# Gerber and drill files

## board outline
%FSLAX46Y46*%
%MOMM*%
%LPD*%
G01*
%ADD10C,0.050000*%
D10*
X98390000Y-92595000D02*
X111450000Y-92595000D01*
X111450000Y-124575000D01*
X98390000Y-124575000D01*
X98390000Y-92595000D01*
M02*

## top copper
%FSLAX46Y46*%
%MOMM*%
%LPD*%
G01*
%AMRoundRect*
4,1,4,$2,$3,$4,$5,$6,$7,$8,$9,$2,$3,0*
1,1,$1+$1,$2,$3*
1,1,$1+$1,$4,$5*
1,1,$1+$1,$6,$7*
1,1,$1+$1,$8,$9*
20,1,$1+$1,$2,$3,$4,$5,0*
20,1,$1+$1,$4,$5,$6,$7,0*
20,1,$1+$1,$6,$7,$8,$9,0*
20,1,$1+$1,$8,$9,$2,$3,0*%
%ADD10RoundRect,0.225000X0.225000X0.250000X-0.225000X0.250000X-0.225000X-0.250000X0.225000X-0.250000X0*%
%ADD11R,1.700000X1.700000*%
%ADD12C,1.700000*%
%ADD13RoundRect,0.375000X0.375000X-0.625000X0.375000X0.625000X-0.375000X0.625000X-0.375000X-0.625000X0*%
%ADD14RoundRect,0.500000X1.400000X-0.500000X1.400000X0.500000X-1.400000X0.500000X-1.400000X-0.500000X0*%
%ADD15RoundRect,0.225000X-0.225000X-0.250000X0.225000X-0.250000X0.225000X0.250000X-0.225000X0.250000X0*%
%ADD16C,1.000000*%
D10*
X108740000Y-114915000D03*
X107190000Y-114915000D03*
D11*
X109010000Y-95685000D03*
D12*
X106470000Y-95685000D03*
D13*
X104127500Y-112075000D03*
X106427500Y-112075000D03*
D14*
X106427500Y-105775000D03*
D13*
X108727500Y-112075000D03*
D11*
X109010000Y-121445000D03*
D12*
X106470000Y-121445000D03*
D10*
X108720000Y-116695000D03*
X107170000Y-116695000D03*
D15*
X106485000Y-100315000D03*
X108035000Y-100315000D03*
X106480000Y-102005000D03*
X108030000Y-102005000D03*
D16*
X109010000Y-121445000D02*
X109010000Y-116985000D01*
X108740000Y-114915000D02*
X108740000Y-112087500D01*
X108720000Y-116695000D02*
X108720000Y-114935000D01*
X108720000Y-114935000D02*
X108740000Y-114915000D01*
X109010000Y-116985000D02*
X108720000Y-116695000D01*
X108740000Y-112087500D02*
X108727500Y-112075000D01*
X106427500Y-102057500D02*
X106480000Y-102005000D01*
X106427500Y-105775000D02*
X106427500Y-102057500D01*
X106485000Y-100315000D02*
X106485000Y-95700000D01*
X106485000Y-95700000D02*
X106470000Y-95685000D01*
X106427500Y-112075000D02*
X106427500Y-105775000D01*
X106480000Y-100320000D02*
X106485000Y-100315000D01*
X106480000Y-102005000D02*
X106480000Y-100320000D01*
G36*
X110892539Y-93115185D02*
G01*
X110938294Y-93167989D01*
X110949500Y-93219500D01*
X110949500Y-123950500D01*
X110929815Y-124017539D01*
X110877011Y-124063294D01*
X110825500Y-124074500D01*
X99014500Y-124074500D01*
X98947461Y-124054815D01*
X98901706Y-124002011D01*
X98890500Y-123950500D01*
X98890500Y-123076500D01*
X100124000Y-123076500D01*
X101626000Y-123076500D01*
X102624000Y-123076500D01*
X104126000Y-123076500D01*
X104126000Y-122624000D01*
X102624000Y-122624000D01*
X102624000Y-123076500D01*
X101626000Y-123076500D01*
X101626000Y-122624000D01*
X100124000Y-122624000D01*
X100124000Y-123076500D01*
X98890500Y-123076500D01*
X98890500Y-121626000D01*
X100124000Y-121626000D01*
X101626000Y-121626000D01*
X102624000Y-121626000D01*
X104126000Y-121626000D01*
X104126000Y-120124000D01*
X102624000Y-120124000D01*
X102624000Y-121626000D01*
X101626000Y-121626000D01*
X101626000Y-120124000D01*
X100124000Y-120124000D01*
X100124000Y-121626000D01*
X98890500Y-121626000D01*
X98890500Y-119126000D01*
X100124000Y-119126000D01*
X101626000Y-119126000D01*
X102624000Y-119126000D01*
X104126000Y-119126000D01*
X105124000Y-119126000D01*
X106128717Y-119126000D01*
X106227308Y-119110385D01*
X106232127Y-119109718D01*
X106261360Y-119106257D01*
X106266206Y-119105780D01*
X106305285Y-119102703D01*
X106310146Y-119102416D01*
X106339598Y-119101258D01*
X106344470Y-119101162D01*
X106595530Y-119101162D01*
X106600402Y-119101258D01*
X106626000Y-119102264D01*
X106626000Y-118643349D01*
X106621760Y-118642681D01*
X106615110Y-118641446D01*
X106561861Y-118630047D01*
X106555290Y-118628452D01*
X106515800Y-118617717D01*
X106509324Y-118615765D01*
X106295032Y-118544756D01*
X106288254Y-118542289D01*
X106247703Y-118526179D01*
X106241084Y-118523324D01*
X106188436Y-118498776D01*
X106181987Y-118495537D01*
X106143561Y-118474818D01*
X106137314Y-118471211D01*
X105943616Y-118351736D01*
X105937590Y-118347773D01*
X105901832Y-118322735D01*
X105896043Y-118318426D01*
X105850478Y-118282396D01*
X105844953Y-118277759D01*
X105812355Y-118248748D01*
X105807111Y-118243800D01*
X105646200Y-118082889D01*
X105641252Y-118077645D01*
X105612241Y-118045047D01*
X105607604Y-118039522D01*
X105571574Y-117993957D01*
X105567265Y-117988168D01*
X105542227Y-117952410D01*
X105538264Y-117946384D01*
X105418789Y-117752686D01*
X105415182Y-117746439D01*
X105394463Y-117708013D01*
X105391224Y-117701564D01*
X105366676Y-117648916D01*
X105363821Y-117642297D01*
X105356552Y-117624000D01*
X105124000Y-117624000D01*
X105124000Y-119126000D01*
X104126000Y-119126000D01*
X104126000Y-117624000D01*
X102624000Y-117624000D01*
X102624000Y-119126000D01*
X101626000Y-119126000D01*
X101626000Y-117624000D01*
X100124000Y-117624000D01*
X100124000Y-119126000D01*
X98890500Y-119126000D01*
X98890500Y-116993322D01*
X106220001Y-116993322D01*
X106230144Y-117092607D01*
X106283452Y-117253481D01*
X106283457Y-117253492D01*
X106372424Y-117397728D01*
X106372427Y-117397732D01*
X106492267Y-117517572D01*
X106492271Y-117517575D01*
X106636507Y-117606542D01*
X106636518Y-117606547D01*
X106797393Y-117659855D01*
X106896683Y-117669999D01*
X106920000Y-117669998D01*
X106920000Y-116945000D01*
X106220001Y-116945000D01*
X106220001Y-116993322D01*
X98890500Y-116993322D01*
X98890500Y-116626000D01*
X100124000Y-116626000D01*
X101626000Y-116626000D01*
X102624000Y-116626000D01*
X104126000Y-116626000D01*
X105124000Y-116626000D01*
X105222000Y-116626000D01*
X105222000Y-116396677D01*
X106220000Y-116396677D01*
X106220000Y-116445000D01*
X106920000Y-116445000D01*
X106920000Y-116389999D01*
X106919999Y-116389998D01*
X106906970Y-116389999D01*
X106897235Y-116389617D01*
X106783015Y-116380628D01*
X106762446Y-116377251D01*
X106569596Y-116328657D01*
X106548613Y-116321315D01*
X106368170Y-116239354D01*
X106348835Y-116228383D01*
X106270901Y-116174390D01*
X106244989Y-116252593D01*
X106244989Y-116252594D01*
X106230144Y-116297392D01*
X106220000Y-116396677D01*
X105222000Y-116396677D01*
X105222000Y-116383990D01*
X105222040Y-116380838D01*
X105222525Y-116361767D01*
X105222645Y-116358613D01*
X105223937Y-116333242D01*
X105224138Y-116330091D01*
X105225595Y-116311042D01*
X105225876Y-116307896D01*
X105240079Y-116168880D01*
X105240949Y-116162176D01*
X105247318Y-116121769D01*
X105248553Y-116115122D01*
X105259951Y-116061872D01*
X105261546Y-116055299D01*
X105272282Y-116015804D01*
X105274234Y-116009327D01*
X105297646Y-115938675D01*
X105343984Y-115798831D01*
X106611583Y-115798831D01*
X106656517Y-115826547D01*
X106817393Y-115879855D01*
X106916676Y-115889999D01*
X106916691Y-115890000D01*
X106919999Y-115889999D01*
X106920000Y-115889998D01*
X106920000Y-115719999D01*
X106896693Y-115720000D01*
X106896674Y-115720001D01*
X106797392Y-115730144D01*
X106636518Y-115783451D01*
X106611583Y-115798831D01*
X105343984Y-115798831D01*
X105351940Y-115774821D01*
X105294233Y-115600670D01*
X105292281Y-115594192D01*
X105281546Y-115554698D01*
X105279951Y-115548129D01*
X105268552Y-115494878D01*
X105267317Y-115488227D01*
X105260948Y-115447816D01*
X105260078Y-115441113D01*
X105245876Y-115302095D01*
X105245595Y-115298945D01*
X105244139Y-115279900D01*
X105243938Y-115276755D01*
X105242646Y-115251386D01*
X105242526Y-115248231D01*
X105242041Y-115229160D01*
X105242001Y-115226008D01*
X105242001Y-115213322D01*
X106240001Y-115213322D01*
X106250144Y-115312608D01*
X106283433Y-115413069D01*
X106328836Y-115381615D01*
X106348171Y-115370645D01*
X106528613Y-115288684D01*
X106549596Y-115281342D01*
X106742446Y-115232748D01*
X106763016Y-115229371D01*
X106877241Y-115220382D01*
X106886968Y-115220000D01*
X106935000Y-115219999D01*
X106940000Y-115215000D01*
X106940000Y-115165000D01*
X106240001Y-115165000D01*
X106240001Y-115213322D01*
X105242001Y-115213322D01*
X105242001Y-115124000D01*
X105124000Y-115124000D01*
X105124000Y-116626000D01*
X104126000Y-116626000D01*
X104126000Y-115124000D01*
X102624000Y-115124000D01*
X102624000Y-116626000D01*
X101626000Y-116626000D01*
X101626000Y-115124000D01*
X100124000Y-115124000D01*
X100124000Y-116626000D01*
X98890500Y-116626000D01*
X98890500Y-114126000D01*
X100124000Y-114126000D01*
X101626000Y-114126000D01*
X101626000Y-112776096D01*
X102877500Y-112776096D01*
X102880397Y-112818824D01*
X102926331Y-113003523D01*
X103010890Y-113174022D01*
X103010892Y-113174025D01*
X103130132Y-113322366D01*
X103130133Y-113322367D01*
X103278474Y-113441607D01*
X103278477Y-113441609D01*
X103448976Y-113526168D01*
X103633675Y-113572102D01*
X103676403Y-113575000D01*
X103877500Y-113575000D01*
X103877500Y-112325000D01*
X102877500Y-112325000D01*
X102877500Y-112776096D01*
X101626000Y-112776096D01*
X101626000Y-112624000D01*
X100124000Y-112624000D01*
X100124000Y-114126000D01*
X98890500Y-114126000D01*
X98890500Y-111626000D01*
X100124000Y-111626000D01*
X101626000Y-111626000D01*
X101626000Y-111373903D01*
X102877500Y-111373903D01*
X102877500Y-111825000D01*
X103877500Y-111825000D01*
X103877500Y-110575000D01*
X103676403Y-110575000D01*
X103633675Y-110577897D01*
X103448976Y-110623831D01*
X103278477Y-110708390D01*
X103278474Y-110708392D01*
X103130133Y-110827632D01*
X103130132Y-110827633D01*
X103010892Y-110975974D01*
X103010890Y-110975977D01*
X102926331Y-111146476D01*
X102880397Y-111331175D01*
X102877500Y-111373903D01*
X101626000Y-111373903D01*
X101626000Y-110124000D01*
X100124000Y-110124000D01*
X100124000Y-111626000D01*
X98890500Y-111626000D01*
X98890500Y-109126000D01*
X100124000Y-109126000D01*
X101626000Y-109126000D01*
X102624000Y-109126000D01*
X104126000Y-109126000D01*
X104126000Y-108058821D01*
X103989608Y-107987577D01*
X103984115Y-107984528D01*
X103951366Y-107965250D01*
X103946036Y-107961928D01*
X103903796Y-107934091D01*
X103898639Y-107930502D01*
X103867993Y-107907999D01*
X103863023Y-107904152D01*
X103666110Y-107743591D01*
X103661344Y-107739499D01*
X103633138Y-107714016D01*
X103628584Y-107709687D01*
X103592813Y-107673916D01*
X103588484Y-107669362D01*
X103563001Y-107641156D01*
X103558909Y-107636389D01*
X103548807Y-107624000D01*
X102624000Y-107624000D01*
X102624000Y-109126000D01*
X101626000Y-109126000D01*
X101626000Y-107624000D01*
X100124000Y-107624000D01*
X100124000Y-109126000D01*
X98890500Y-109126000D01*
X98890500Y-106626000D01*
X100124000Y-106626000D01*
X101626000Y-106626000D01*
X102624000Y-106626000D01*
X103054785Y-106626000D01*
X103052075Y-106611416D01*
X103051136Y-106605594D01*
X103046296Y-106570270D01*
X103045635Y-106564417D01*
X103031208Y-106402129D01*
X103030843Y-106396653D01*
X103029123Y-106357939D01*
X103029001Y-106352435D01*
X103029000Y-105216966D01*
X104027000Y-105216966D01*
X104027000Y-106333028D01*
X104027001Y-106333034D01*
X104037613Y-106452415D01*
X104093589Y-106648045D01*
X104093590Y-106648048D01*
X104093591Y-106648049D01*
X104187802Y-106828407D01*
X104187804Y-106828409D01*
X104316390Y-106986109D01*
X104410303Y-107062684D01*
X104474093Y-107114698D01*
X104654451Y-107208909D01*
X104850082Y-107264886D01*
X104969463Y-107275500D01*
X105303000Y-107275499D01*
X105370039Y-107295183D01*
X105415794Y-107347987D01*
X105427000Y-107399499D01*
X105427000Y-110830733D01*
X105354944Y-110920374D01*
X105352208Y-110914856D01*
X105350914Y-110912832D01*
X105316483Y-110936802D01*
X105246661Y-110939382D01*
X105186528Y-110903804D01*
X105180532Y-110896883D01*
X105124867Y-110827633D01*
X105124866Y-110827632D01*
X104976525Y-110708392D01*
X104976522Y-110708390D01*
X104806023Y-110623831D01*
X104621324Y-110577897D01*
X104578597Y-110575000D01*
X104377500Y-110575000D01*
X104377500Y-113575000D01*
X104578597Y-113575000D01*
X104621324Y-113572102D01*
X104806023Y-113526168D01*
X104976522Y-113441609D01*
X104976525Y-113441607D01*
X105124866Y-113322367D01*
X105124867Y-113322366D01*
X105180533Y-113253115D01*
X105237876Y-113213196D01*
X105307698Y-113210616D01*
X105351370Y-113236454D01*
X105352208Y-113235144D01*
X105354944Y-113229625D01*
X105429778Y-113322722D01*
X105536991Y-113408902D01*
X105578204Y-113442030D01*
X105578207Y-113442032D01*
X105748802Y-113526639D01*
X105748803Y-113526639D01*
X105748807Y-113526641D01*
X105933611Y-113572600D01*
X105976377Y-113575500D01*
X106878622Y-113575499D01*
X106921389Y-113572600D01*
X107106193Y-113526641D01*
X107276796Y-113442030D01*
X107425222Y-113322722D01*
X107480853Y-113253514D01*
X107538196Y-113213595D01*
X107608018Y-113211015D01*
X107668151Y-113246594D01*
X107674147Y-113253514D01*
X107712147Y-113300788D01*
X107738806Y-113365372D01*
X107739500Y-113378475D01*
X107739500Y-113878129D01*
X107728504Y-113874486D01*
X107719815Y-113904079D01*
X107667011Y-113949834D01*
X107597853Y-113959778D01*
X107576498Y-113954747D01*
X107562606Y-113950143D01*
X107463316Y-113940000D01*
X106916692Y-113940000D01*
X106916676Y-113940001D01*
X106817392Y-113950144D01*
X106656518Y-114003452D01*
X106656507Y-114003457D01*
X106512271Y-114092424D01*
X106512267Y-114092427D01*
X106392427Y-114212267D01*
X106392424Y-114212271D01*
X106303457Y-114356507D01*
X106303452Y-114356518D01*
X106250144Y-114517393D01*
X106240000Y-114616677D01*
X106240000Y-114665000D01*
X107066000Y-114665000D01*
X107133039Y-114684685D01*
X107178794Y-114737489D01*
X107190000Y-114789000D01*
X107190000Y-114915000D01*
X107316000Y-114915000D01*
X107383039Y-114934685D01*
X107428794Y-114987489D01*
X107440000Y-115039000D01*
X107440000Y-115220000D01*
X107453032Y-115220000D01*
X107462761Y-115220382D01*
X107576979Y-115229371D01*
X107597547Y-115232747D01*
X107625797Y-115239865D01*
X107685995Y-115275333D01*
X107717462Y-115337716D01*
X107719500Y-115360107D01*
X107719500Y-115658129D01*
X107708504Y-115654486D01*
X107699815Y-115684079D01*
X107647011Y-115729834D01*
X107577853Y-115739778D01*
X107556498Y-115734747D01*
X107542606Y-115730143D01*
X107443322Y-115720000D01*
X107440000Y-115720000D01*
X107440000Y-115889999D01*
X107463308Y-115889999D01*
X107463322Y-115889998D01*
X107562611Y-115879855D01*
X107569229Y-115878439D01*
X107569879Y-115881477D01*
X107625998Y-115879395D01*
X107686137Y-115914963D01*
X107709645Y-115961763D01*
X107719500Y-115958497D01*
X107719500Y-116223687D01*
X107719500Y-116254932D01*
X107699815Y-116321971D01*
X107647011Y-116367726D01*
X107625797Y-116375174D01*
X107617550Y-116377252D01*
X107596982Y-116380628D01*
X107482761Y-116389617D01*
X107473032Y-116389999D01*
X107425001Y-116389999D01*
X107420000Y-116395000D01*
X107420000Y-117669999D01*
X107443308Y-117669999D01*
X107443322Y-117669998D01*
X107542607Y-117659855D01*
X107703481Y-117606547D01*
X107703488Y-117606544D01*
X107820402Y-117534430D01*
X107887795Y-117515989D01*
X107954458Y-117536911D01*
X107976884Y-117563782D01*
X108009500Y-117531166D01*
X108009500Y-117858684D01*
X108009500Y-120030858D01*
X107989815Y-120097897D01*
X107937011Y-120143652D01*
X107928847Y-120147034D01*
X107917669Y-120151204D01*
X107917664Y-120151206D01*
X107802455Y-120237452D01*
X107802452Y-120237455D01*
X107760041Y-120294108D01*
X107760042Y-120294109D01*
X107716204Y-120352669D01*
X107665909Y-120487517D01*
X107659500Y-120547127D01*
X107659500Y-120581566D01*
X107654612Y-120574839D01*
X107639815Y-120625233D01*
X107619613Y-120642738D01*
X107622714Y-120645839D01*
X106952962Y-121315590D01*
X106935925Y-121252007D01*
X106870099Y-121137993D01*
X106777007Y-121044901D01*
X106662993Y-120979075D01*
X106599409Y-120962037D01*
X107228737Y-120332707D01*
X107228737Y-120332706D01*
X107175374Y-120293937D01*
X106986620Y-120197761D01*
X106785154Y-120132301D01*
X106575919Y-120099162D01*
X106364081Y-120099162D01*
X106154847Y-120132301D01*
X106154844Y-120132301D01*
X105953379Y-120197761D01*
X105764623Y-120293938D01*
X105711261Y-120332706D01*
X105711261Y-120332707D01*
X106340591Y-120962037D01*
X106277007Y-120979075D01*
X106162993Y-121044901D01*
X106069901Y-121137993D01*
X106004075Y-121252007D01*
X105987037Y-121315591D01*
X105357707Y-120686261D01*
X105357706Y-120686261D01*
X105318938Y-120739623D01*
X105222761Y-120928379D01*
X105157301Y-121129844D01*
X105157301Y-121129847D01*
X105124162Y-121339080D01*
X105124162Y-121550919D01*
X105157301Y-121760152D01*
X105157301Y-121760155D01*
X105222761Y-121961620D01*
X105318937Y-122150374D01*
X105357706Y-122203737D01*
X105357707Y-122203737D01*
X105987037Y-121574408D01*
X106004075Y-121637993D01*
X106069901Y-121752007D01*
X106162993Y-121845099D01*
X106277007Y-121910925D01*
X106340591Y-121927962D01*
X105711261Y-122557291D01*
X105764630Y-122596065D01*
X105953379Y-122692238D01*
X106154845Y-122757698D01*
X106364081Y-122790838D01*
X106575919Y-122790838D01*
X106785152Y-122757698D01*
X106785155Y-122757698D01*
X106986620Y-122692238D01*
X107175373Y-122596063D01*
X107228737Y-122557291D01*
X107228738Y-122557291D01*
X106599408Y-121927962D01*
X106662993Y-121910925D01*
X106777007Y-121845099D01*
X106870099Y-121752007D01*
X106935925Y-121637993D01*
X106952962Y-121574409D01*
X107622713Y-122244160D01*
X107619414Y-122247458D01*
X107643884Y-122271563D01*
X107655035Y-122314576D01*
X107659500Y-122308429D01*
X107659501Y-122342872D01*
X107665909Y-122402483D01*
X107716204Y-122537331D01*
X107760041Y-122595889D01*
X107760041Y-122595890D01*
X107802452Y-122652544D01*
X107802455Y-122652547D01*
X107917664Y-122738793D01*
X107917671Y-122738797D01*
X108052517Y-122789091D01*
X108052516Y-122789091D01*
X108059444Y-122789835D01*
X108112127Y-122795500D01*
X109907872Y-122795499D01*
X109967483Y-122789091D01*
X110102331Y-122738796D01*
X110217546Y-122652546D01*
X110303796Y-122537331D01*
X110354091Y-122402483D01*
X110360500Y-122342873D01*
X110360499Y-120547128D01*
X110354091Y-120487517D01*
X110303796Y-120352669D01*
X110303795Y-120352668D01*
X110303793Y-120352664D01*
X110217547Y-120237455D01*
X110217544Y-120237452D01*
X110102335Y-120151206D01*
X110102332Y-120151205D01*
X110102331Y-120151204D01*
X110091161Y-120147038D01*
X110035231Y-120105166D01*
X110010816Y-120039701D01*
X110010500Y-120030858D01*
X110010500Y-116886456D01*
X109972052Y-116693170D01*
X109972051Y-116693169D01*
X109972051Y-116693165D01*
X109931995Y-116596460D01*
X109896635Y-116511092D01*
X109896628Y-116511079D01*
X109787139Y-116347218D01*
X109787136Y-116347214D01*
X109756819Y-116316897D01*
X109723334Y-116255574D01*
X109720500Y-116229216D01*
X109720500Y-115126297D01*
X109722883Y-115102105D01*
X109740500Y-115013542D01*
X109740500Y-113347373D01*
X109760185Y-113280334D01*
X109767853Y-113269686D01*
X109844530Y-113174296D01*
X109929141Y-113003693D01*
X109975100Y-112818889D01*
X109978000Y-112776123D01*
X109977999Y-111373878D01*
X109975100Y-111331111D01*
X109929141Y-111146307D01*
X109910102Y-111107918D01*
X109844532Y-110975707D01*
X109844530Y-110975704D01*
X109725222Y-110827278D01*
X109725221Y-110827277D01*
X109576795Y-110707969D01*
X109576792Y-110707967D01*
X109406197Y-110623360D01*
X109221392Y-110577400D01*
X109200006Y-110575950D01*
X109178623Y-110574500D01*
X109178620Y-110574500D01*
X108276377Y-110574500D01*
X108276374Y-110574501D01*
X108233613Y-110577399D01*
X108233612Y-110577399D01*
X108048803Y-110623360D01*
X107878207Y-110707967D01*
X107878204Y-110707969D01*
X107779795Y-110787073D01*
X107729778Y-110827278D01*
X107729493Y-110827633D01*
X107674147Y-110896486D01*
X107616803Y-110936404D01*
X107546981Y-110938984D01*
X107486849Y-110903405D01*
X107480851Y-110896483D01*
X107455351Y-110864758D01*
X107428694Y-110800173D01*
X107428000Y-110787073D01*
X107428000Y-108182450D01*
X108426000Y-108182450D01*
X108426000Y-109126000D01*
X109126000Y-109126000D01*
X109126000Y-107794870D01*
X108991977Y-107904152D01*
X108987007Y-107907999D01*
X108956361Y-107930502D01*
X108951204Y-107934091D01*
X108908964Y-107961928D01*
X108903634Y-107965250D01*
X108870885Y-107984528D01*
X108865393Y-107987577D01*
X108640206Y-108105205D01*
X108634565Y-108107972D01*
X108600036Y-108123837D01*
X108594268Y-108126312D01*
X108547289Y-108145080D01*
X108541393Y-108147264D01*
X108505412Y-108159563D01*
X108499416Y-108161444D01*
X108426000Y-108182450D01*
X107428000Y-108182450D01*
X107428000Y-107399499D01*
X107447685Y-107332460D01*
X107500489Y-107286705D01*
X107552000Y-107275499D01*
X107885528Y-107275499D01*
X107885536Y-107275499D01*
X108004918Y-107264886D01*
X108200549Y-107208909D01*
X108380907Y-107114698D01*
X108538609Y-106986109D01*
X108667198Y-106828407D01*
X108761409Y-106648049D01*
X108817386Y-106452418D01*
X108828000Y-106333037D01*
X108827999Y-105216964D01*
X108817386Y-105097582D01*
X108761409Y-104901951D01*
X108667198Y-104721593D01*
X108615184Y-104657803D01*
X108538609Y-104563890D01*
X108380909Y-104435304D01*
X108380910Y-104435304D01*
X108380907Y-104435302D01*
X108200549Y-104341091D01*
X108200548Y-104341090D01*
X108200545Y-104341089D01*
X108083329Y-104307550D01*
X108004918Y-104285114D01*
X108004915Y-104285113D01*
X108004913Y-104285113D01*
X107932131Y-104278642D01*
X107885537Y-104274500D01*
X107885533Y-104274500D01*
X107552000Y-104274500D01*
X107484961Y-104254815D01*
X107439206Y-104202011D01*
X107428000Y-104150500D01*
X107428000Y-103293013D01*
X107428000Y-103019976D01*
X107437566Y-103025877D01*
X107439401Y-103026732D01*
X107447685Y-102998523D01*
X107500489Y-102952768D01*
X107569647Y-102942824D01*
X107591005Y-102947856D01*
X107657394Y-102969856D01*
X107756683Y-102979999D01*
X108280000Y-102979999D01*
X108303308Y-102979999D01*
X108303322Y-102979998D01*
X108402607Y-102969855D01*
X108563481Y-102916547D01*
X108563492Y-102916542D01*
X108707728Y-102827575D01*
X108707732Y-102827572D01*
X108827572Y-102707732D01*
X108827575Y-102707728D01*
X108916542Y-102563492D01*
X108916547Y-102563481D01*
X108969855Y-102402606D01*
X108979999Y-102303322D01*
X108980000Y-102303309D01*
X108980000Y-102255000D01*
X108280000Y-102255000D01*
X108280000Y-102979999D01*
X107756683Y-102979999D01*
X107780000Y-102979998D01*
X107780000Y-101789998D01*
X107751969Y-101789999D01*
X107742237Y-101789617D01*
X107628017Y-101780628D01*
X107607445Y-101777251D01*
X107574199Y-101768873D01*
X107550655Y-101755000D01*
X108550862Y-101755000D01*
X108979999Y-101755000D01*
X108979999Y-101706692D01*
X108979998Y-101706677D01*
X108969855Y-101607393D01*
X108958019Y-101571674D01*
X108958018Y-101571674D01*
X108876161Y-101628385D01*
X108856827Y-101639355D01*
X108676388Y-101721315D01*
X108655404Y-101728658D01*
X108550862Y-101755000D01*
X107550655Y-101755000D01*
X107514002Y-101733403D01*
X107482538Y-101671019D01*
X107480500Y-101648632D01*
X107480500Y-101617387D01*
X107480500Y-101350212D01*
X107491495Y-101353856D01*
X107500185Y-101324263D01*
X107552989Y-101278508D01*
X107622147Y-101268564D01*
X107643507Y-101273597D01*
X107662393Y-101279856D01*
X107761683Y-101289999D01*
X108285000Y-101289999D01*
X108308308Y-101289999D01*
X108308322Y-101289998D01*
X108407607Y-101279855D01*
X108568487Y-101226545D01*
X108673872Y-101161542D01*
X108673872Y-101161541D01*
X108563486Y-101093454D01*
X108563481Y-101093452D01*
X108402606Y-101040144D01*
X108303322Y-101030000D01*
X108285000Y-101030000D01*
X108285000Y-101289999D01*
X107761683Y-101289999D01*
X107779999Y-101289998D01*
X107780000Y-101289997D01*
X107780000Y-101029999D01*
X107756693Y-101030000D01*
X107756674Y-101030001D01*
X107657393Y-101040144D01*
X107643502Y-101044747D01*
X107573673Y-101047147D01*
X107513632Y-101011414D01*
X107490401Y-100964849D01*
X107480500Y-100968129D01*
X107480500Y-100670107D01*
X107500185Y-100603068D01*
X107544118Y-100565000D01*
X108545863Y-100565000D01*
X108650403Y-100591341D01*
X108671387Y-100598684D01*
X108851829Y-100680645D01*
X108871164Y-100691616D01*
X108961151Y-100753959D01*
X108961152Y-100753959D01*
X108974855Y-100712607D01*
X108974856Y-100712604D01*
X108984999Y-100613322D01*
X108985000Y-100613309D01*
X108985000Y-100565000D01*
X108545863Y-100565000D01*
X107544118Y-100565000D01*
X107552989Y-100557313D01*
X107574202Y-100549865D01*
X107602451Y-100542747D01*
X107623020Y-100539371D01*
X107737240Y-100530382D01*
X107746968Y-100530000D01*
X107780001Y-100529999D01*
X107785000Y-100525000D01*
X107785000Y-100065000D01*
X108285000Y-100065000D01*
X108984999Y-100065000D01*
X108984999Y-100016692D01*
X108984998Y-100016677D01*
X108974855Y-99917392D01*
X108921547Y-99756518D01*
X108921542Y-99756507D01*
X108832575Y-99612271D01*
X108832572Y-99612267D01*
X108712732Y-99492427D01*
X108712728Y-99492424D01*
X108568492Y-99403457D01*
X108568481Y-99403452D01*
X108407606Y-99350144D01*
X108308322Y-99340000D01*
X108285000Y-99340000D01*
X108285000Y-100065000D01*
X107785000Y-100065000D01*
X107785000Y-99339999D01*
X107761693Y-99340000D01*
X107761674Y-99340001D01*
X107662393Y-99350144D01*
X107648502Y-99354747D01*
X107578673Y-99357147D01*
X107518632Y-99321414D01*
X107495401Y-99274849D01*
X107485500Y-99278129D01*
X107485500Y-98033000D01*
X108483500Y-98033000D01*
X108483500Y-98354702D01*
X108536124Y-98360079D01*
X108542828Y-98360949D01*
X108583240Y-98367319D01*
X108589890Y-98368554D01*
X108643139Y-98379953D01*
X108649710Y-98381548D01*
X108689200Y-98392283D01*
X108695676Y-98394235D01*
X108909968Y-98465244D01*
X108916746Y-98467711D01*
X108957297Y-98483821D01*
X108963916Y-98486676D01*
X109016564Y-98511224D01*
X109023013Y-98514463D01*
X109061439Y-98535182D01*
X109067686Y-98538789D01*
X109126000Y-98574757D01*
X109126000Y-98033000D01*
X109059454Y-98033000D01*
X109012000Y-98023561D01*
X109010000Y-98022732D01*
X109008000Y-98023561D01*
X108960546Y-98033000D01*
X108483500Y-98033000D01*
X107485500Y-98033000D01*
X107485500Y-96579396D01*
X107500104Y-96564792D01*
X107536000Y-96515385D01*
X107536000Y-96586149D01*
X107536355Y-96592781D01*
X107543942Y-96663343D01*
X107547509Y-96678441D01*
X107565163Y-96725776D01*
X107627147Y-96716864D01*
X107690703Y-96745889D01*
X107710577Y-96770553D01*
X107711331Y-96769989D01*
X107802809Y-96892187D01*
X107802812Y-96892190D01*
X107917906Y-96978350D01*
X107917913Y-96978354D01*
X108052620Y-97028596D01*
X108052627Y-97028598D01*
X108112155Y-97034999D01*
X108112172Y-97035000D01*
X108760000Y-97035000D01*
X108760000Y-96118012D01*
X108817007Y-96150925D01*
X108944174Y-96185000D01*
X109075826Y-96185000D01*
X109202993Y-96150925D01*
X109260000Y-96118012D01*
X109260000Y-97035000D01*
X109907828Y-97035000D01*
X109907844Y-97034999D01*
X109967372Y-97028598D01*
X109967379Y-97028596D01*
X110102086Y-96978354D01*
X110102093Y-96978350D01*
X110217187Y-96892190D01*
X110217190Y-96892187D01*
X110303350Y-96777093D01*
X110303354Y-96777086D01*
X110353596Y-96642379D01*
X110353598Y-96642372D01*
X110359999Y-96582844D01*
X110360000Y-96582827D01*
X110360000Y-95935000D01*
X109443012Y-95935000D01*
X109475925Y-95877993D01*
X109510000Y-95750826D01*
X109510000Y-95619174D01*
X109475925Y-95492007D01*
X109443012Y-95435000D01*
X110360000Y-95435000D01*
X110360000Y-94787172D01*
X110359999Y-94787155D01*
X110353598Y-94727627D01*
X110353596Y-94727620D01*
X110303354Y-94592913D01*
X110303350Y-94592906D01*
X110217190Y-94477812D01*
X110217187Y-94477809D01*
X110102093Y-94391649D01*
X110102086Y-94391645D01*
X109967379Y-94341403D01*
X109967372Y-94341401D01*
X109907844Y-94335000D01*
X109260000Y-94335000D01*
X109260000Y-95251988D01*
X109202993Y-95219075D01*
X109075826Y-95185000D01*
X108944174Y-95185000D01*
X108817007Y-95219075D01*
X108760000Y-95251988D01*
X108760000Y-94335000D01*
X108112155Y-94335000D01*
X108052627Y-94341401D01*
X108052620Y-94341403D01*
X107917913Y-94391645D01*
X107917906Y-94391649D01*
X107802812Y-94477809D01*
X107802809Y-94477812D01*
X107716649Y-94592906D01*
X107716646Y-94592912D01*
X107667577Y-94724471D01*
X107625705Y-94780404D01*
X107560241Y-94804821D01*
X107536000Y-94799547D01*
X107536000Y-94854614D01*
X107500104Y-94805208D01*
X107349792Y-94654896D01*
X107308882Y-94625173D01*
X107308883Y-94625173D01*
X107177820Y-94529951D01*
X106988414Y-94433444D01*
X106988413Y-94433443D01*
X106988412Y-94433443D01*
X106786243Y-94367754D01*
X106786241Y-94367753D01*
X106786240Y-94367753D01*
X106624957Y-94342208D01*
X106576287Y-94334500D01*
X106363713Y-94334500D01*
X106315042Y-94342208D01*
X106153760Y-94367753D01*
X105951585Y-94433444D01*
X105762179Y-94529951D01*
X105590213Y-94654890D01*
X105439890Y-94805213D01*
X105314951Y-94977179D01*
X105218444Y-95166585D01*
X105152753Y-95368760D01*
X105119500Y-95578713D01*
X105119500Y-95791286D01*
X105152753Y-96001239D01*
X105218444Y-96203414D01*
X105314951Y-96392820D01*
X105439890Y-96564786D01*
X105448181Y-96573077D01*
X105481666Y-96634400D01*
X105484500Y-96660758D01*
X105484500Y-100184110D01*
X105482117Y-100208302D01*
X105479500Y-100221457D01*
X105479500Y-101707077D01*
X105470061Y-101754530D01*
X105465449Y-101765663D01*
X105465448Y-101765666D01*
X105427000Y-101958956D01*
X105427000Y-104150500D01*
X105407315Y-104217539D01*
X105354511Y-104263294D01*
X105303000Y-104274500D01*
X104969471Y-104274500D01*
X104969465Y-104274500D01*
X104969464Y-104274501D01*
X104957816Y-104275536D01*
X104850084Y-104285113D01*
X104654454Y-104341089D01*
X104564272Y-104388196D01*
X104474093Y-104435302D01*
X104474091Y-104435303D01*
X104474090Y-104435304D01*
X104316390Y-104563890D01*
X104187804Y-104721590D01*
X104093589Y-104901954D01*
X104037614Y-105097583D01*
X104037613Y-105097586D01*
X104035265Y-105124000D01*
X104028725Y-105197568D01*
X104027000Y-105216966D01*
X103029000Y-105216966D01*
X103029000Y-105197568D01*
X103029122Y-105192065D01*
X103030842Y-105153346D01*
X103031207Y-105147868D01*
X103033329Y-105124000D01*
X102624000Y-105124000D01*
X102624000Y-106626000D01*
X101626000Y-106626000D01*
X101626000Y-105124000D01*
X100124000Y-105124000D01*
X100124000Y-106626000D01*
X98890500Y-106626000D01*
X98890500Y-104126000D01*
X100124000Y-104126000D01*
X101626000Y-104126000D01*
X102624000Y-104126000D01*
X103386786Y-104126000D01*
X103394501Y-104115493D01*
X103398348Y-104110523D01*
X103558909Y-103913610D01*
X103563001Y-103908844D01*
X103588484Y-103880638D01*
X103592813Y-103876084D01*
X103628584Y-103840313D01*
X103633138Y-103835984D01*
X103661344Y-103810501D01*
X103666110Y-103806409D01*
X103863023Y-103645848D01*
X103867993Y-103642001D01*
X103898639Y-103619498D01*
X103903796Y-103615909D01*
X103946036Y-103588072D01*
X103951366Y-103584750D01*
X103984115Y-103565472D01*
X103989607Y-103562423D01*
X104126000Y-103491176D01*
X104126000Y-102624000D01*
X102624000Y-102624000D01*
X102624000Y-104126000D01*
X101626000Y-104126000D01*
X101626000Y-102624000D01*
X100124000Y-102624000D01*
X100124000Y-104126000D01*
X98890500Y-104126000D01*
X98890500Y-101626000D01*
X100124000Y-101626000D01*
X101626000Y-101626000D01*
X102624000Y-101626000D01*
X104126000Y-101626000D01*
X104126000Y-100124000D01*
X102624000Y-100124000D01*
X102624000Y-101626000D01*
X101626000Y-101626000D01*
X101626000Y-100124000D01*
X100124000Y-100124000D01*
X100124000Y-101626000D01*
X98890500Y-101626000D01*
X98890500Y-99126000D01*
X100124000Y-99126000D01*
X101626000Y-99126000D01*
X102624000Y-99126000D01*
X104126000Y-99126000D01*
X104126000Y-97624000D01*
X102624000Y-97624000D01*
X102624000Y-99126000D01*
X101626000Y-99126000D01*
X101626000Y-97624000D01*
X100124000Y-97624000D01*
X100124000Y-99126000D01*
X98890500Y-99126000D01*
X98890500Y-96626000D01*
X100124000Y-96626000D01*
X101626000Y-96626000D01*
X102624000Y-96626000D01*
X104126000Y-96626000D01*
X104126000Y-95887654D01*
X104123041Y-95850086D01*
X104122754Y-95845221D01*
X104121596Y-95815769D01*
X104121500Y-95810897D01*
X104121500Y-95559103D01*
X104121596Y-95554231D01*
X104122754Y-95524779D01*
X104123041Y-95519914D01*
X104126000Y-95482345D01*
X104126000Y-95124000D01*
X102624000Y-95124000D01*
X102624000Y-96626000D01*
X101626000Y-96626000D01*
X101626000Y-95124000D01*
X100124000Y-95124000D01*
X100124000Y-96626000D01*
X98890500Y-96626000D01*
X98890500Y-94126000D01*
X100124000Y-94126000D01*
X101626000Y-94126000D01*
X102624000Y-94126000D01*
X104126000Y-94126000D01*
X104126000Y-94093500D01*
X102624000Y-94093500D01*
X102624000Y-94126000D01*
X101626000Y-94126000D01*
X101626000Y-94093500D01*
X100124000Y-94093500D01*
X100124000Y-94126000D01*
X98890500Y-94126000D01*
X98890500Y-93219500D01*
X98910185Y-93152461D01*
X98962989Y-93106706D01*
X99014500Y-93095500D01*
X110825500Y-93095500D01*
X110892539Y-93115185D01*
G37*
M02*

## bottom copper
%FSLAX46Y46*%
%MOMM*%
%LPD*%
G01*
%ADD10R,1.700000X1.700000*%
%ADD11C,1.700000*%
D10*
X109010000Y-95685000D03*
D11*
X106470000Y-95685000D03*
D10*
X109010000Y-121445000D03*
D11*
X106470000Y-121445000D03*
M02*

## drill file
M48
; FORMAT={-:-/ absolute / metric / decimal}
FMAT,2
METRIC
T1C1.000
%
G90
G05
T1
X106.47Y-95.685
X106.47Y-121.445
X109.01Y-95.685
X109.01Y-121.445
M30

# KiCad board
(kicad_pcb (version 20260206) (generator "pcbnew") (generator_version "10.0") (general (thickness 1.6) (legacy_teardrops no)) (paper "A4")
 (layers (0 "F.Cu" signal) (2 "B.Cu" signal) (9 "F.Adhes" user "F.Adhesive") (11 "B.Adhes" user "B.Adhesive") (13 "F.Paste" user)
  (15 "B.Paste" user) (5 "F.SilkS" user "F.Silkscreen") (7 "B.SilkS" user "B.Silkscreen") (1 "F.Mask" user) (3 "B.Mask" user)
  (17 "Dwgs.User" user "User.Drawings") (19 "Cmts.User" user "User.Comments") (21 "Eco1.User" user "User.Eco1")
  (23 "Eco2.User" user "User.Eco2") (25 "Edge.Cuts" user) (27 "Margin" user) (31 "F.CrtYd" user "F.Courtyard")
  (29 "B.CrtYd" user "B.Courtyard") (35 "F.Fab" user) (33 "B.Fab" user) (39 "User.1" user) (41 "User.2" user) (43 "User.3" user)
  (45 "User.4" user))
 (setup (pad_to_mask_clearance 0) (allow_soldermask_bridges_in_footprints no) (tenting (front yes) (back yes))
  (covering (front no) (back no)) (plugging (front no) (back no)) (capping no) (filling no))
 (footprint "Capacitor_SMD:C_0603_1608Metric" (layer "F.Cu") (at 107.965 114.915 180)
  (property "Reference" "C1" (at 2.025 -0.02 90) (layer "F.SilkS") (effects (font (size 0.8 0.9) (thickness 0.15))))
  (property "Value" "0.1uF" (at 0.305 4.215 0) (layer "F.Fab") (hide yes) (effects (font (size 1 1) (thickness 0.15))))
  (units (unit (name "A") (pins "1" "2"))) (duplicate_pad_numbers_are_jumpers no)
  (pad "1" smd roundrect (at -0.775 0 180) (size 0.9 0.95) (layers "F.Cu" "F.Mask" "F.Paste") (roundrect_rratio 0.25) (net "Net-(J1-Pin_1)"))
  (pad "2" smd roundrect (at 0.775 0 180) (size 0.9 0.95) (layers "F.Cu" "F.Mask" "F.Paste") (roundrect_rratio 0.25) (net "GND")))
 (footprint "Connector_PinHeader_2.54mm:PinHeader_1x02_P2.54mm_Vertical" (layer "F.Cu") (at 109.01 95.685 -90)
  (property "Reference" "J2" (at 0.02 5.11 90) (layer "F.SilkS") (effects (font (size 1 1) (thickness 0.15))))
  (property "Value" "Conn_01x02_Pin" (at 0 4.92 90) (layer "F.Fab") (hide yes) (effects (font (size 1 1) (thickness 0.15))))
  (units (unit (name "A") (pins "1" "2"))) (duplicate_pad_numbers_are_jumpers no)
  (pad "1" thru_hole rect (at 0 0 270) (size 1.7 1.7) (drill 1) (layers "*.Cu" "*.Mask") (remove_unused_layers no) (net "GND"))
  (pad "2" thru_hole circle (at 0 2.54 270) (size 1.7 1.7) (drill 1) (layers "*.Cu" "*.Mask") (remove_unused_layers no)
   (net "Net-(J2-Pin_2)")))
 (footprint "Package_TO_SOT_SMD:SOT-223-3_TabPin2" (layer "F.Cu") (at 106.4275 108.925 90)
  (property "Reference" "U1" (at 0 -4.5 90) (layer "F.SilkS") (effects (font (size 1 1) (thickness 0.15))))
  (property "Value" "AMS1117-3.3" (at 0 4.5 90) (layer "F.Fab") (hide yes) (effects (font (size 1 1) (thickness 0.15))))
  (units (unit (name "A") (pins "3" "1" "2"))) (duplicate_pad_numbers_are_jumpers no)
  (pad "1" smd roundrect (at -3.15 -2.3 90) (size 2 1.5) (layers "F.Cu" "F.Mask" "F.Paste") (roundrect_rratio 0.25) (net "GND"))
  (pad "2" smd roundrect (at -3.15 0 90) (size 2 1.5) (layers "F.Cu" "F.Mask" "F.Paste") (roundrect_rratio 0.25) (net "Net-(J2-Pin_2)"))
  (pad "2" smd roundrect (at 3.15 0 90) (size 2 3.8) (layers "F.Cu" "F.Mask" "F.Paste") (roundrect_rratio 0.25) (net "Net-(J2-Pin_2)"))
  (pad "3" smd roundrect (at -3.15 2.3 90) (size 2 1.5) (layers "F.Cu" "F.Mask" "F.Paste") (roundrect_rratio 0.25) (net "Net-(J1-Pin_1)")))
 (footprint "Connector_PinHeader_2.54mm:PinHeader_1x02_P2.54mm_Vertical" (layer "F.Cu") (at 109.01 121.445 -90)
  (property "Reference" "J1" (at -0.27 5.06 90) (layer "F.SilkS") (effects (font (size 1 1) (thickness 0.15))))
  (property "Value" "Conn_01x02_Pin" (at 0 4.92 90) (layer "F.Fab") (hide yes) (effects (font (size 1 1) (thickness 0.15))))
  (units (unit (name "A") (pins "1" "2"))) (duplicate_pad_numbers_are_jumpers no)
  (pad "1" thru_hole rect (at 0 0 270) (size 1.7 1.7) (drill 1) (layers "*.Cu" "*.Mask") (remove_unused_layers no) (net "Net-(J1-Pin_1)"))
  (pad "2" thru_hole circle (at 0 2.54 270) (size 1.7 1.7) (drill 1) (layers "*.Cu" "*.Mask") (remove_unused_layers no) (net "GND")))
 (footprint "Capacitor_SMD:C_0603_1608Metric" (layer "F.Cu") (at 107.945 116.695 180)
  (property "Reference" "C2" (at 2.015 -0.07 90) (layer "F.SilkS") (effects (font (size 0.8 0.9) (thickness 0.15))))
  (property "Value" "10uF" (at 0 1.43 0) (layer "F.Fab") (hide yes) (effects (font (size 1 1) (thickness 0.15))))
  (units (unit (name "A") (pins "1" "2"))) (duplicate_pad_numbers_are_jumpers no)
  (pad "1" smd roundrect (at -0.775 0 180) (size 0.9 0.95) (layers "F.Cu" "F.Mask" "F.Paste") (roundrect_rratio 0.25) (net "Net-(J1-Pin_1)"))
  (pad "2" smd roundrect (at 0.775 0 180) (size 0.9 0.95) (layers "F.Cu" "F.Mask" "F.Paste") (roundrect_rratio 0.25) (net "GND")))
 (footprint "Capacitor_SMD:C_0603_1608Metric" (layer "F.Cu") (at 107.26 100.315)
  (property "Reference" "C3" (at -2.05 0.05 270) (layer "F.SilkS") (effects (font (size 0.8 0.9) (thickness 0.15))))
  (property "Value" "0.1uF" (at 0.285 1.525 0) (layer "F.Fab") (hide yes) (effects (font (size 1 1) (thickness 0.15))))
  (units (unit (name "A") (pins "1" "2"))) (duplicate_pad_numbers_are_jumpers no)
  (pad "1" smd roundrect (at -0.775 0) (size 0.9 0.95) (layers "F.Cu" "F.Mask" "F.Paste") (roundrect_rratio 0.25) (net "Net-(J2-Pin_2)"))
  (pad "2" smd roundrect (at 0.775 0) (size 0.9 0.95) (layers "F.Cu" "F.Mask" "F.Paste") (roundrect_rratio 0.25) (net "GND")))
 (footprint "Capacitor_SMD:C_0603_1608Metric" (layer "F.Cu") (at 107.255 102.005)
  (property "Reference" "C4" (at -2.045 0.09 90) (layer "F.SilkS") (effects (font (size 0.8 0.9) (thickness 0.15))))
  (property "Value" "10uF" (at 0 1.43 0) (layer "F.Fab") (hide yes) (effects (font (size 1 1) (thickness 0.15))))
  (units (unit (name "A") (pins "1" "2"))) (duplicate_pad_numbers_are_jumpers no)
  (pad "1" smd roundrect (at -0.775 0) (size 0.9 0.95) (layers "F.Cu" "F.Mask" "F.Paste") (roundrect_rratio 0.25) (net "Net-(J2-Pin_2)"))
  (pad "2" smd roundrect (at 0.775 0) (size 0.9 0.95) (layers "F.Cu" "F.Mask" "F.Paste") (roundrect_rratio 0.25) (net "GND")))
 (gr_rect (start 98.39 92.595) (end 111.45 124.575) (stroke (width 0.05) (type default)) (fill no) (layer "Edge.Cuts"))
 (segment (start 109.01 121.445) (end 109.01 116.985) (width 1) (layer "F.Cu") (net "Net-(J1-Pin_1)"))
 (segment (start 108.74 114.915) (end 108.74 112.0875) (width 1) (layer "F.Cu") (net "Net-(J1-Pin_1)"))
 (segment (start 108.72 116.695) (end 108.72 114.935) (width 1) (layer "F.Cu") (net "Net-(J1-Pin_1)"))
 (segment (start 108.72 114.935) (end 108.74 114.915) (width 1) (layer "F.Cu") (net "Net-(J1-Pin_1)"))
 (segment (start 109.01 116.985) (end 108.72 116.695) (width 1) (layer "F.Cu") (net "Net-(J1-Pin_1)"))
 (segment (start 108.74 112.0875) (end 108.7275 112.075) (width 1) (layer "F.Cu") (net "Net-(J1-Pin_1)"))
 (segment (start 106.4275 102.0575) (end 106.48 102.005) (width 1) (layer "F.Cu") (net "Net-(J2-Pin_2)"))
 (segment (start 106.4275 105.775) (end 106.4275 102.0575) (width 1) (layer "F.Cu") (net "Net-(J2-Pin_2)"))
 (segment (start 106.485 100.315) (end 106.485 95.7) (width 1) (layer "F.Cu") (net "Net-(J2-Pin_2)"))
 (segment (start 106.485 95.7) (end 106.47 95.685) (width 1) (layer "F.Cu") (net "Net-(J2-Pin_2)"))
 (segment (start 106.4275 112.075) (end 106.4275 105.775) (width 1) (layer "F.Cu") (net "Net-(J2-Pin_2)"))
 (segment (start 106.48 100.32) (end 106.485 100.315) (width 1) (layer "F.Cu") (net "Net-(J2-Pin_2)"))
 (segment (start 106.48 102.005) (end 106.48 100.32) (width 1) (layer "F.Cu") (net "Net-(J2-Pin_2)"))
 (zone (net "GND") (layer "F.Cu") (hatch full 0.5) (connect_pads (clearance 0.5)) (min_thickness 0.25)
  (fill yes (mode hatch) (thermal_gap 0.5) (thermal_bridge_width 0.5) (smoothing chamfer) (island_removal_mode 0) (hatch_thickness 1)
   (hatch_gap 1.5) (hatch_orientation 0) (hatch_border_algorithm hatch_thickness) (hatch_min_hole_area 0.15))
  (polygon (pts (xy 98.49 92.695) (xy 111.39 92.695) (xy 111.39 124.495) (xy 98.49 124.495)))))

